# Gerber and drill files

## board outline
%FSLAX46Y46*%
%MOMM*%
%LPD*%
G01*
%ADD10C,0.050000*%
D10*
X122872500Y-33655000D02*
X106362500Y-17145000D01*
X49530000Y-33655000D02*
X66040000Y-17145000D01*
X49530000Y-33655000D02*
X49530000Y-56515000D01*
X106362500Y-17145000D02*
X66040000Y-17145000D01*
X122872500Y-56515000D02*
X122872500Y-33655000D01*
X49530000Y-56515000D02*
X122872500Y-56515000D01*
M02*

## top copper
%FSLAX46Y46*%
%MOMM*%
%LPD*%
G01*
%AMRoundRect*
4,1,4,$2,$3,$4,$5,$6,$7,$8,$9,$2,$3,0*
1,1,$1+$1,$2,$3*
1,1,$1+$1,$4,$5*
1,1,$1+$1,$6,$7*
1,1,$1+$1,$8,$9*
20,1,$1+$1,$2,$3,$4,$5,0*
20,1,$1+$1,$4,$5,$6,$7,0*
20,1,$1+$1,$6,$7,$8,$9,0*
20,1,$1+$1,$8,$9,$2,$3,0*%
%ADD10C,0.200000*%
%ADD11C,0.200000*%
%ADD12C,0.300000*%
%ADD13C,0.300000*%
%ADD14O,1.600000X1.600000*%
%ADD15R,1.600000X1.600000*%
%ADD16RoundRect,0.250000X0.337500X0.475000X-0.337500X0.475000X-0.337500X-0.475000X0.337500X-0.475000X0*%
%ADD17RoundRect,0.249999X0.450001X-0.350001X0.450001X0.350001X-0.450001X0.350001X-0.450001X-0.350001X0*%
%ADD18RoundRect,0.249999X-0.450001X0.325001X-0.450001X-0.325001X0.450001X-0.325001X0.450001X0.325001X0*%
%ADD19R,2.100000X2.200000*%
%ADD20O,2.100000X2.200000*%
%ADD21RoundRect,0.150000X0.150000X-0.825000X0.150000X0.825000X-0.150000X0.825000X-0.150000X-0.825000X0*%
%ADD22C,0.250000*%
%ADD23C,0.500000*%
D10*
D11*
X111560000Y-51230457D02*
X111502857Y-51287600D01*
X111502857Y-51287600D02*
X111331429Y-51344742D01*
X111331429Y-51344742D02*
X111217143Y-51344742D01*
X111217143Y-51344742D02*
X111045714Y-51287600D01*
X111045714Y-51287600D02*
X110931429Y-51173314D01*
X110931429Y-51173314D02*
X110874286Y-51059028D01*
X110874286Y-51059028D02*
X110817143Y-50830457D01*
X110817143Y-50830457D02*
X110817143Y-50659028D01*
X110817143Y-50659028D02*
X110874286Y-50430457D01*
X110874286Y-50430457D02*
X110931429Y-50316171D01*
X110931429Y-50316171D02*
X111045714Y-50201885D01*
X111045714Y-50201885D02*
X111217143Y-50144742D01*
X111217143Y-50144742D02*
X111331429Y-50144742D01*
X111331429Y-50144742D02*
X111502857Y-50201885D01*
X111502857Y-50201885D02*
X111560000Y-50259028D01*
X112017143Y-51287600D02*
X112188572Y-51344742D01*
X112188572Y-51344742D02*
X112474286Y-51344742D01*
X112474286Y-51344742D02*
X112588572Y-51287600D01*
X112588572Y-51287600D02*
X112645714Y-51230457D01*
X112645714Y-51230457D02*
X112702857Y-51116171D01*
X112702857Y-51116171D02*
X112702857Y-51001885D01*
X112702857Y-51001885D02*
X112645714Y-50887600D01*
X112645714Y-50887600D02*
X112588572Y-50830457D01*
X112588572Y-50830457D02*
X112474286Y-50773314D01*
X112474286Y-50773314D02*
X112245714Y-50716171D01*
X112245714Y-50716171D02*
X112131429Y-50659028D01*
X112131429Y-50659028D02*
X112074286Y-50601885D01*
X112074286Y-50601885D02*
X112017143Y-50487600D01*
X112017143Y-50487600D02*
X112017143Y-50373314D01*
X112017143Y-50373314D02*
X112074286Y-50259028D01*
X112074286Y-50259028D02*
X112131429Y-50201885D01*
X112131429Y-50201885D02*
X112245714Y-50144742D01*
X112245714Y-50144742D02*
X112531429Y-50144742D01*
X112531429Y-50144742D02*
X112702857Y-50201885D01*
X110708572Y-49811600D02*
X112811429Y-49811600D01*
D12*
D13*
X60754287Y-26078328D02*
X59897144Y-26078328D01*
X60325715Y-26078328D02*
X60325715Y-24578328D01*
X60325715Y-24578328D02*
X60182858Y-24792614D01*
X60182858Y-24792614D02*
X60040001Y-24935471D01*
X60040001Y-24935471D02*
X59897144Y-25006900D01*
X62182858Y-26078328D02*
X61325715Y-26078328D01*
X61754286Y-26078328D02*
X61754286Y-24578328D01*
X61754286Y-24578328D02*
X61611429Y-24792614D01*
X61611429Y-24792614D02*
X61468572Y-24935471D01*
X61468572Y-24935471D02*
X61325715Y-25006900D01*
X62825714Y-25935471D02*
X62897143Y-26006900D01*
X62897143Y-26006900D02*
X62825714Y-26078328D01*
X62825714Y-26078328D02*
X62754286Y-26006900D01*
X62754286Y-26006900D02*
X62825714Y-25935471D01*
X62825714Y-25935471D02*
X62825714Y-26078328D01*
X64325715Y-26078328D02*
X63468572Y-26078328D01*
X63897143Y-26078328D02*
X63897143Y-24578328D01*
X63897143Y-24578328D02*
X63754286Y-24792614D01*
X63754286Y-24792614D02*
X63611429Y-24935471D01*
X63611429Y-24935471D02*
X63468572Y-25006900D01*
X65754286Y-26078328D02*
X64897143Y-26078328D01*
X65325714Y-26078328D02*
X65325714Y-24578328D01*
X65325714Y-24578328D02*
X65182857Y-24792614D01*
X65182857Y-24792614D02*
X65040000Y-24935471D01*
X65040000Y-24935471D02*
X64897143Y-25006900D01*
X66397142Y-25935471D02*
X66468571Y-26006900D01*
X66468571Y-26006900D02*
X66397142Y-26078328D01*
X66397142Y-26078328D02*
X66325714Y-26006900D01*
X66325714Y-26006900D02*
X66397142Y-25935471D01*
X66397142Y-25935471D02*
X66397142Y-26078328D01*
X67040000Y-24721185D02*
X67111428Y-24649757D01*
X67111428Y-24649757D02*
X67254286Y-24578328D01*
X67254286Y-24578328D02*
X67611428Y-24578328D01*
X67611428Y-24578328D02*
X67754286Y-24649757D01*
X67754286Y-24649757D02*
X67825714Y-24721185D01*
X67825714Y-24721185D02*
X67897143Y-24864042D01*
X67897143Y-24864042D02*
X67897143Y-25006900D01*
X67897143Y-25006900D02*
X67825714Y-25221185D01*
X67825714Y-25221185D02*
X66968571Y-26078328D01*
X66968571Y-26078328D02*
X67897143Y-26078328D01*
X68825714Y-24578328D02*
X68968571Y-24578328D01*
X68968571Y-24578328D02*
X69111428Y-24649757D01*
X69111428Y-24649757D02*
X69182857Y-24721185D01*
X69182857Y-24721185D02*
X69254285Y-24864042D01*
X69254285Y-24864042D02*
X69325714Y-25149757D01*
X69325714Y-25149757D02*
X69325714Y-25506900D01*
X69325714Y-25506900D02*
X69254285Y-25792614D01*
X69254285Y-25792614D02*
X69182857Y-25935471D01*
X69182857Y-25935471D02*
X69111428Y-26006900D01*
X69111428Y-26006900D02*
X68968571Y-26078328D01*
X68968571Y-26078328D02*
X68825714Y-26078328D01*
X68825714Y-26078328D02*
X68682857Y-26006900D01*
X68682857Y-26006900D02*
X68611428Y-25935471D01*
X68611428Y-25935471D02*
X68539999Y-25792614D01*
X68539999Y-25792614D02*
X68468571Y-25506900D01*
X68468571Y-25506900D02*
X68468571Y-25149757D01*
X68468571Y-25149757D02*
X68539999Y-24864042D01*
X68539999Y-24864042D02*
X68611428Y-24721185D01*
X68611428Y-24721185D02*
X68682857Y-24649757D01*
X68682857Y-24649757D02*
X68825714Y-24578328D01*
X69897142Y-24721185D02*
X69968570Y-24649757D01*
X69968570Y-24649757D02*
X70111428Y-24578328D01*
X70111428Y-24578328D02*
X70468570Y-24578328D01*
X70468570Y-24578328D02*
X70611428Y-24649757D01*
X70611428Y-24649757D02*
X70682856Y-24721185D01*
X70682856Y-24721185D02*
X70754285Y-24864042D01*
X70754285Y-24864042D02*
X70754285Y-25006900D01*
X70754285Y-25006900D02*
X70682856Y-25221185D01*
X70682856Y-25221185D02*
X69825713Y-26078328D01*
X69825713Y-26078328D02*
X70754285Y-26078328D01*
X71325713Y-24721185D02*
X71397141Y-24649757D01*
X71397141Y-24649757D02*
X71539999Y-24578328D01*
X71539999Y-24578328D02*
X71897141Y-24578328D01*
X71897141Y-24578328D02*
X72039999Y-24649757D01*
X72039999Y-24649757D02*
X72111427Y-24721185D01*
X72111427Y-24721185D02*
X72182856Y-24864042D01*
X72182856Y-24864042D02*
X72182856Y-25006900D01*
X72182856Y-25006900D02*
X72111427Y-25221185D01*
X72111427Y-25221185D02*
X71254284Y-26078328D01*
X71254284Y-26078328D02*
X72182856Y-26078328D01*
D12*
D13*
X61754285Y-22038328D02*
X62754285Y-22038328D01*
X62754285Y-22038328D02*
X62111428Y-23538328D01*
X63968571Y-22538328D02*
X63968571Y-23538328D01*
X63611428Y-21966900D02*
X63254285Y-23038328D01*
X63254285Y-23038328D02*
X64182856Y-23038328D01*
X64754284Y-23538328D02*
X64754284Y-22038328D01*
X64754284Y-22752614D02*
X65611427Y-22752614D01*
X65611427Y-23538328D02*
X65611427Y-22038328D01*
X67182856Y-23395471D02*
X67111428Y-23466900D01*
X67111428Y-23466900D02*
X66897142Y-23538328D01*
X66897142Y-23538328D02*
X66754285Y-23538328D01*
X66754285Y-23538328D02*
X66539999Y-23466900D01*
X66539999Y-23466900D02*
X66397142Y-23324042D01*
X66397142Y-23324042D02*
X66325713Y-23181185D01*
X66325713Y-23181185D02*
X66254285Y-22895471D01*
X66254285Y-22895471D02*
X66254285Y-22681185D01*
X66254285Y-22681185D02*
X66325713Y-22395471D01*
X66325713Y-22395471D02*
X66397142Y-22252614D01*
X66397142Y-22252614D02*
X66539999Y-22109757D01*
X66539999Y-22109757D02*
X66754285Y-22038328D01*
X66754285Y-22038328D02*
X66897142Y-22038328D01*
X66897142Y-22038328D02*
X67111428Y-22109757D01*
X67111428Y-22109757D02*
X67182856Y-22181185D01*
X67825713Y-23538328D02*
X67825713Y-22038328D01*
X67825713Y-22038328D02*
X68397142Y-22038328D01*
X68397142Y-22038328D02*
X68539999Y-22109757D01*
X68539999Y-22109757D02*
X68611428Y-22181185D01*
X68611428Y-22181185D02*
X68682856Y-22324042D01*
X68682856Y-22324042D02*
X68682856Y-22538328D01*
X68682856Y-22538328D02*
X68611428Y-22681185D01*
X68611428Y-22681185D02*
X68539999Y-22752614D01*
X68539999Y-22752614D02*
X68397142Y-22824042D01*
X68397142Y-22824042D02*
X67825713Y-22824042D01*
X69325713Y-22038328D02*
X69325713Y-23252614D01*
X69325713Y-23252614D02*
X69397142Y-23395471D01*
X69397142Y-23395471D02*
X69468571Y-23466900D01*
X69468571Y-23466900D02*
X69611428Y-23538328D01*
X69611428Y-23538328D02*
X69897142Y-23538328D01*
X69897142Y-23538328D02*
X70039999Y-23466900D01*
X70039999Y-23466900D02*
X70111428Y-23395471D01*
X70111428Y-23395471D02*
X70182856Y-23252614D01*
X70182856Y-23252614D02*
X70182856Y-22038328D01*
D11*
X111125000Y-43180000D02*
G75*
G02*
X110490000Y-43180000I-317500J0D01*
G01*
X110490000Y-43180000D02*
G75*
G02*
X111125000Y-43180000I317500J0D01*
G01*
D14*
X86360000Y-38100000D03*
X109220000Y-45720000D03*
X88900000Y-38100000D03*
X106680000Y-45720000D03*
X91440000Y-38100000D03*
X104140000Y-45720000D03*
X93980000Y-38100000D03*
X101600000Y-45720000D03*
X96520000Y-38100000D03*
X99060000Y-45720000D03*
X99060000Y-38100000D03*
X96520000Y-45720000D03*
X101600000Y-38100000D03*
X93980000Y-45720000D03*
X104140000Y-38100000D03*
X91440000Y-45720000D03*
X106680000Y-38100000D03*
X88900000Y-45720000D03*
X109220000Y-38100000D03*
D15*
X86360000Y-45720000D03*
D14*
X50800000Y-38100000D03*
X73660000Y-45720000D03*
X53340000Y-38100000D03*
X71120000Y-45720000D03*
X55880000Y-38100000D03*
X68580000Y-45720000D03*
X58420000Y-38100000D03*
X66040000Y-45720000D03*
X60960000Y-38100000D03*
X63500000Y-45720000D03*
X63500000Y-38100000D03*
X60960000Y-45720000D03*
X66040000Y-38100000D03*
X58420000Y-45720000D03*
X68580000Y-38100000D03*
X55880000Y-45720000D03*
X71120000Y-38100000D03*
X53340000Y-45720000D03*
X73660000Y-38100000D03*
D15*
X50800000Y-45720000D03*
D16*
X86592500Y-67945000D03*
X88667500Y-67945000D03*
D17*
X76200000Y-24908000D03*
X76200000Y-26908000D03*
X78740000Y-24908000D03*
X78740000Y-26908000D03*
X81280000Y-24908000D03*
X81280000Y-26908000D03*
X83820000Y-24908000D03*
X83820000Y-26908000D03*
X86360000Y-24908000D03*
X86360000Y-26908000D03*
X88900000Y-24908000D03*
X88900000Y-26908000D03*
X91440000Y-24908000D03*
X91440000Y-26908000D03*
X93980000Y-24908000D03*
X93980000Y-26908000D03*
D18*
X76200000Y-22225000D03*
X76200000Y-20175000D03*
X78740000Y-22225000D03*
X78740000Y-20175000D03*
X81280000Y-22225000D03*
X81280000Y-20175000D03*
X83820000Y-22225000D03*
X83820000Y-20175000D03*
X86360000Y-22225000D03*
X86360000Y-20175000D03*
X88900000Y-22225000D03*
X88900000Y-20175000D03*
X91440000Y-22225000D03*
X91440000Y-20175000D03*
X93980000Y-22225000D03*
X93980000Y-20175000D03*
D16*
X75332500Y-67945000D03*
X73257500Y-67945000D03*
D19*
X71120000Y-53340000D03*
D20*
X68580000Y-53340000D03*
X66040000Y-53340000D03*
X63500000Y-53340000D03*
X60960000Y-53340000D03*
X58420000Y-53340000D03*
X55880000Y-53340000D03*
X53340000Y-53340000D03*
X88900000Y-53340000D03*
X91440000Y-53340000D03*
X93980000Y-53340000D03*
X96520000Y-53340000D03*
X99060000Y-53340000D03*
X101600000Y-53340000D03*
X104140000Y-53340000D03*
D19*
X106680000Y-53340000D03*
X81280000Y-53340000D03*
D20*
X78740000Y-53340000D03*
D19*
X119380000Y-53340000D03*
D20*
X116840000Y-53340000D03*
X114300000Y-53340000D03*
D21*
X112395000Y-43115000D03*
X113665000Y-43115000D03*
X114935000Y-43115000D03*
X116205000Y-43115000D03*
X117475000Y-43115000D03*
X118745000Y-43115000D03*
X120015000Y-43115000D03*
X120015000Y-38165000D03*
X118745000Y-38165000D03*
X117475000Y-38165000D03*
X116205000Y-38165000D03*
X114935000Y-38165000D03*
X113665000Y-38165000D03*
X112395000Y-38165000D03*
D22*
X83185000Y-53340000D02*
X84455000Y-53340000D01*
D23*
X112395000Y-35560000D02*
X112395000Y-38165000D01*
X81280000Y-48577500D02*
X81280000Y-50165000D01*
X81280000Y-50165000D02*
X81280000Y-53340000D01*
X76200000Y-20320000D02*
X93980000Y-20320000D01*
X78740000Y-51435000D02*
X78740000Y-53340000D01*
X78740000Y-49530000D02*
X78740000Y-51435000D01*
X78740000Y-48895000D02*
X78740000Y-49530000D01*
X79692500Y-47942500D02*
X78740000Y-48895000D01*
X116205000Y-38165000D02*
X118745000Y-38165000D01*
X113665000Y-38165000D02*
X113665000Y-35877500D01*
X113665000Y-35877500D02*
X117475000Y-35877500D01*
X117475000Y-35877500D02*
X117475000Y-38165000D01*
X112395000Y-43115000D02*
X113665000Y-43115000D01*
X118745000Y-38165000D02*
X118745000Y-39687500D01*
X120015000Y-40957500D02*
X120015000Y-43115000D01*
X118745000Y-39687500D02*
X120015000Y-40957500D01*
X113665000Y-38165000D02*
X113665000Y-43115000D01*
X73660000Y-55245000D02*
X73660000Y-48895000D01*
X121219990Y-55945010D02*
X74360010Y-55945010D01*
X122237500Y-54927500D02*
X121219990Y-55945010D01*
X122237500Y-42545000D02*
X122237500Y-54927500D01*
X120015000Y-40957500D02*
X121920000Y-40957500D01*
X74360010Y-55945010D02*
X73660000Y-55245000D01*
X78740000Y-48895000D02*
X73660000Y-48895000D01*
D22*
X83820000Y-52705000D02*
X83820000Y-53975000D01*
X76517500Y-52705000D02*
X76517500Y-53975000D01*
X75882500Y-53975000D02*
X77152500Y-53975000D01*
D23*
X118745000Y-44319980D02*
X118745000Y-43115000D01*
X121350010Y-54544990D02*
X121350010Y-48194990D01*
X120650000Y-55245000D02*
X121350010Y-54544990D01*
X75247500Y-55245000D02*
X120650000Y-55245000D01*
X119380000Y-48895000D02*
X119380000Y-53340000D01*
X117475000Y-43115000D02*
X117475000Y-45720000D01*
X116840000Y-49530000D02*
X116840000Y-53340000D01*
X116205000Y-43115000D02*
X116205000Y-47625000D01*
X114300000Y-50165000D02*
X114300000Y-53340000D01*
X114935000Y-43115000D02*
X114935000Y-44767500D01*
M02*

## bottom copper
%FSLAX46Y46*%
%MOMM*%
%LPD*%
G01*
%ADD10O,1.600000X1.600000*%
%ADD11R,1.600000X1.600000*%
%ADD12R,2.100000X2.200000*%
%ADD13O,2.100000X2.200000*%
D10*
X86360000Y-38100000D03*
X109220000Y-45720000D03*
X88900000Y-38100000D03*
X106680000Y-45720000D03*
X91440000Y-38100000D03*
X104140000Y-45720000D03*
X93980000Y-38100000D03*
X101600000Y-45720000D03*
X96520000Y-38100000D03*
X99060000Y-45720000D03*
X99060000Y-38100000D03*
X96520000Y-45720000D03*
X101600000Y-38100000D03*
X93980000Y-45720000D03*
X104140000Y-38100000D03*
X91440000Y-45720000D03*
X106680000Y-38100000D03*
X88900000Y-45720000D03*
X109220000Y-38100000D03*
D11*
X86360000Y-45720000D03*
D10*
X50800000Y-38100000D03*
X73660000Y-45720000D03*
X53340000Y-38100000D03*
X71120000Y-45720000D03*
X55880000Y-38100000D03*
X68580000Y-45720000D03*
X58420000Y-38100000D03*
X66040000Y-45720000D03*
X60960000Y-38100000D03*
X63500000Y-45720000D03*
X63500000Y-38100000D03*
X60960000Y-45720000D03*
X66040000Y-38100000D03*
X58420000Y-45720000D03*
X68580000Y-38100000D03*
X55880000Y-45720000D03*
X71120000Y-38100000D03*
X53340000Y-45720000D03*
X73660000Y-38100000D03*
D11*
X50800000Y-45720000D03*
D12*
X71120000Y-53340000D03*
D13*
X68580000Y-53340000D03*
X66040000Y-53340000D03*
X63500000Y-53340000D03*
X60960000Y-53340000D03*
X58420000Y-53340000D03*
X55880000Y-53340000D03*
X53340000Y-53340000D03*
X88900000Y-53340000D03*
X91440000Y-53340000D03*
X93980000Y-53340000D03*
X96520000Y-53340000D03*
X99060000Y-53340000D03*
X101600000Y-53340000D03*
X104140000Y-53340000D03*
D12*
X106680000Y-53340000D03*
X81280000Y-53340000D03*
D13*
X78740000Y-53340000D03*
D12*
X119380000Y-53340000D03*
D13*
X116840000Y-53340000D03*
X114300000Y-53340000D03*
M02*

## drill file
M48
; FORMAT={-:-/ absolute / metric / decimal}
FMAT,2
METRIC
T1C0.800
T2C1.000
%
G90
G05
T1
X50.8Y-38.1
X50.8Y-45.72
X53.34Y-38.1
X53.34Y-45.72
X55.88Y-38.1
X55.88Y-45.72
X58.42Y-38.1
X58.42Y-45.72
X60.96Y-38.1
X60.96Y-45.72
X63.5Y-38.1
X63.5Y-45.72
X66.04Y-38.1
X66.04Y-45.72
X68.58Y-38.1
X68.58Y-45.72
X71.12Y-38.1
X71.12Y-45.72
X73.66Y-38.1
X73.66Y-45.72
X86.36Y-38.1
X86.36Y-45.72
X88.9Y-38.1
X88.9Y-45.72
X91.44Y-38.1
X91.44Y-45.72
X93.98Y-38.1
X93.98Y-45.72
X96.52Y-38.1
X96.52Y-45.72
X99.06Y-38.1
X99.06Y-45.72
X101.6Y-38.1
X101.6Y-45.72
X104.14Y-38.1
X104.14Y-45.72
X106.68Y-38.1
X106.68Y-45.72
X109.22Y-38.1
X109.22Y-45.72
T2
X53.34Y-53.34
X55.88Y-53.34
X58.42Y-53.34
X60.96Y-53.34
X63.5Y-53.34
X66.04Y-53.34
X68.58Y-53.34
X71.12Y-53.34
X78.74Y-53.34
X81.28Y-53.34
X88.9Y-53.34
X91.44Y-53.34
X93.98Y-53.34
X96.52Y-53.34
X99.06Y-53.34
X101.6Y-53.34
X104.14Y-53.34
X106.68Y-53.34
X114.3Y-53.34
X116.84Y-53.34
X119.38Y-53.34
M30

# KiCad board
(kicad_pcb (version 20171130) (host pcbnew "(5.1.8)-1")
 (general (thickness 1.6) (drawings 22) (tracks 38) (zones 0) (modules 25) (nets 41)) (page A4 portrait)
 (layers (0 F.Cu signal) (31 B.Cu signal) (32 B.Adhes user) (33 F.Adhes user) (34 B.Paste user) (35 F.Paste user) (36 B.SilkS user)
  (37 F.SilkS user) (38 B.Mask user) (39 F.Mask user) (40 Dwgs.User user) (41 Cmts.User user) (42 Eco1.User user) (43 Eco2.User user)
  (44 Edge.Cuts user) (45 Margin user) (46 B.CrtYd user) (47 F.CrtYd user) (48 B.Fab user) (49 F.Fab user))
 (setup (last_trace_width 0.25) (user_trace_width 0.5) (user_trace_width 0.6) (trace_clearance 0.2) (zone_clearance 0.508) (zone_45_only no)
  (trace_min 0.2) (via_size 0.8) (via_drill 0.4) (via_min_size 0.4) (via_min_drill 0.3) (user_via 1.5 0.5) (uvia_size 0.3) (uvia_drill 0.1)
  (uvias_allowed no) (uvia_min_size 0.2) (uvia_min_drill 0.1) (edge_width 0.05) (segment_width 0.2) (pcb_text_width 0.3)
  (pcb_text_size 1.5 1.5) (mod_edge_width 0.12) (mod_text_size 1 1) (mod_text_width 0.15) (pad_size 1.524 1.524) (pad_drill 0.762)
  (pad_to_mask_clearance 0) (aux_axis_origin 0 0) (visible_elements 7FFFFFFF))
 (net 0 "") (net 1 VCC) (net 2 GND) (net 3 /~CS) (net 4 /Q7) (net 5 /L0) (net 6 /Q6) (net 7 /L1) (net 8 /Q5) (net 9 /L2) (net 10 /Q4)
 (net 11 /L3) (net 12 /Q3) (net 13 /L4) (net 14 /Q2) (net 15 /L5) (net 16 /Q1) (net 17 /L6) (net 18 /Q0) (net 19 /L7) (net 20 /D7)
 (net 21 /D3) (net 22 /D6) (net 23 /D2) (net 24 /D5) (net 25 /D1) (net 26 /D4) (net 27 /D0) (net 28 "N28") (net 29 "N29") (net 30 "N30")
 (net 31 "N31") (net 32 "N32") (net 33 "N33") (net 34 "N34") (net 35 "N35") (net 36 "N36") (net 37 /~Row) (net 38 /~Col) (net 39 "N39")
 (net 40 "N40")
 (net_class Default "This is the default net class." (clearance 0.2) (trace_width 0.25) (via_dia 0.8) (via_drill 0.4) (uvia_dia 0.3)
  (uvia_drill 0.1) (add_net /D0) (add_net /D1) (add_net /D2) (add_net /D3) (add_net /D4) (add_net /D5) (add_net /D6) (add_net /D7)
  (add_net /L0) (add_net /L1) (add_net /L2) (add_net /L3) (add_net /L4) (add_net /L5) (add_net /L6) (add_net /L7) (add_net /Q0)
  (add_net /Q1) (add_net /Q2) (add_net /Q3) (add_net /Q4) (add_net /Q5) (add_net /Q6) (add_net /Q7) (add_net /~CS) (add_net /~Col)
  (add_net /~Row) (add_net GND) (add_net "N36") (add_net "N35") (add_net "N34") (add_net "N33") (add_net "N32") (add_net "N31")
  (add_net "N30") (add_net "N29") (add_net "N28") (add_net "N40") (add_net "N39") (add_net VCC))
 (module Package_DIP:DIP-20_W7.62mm (layer F.Cu) (at 86.36 45.72 90)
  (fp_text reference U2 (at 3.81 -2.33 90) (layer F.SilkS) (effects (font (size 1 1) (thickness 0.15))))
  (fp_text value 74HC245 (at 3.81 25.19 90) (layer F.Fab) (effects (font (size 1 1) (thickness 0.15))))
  (pad 20 thru_hole oval (at 7.62 0 90) (size 1.6 1.6) (drill 0.8) (layers *.Cu *.Mask) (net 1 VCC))
  (pad 10 thru_hole oval (at 0 22.86 90) (size 1.6 1.6) (drill 0.8) (layers *.Cu *.Mask) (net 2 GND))
  (pad 19 thru_hole oval (at 7.62 2.54 90) (size 1.6 1.6) (drill 0.8) (layers *.Cu *.Mask) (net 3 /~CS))
  (pad 9 thru_hole oval (at 0 20.32 90) (size 1.6 1.6) (drill 0.8) (layers *.Cu *.Mask) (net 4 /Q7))
  (pad 18 thru_hole oval (at 7.62 5.08 90) (size 1.6 1.6) (drill 0.8) (layers *.Cu *.Mask) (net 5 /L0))
  (pad 8 thru_hole oval (at 0 17.78 90) (size 1.6 1.6) (drill 0.8) (layers *.Cu *.Mask) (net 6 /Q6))
  (pad 17 thru_hole oval (at 7.62 7.62 90) (size 1.6 1.6) (drill 0.8) (layers *.Cu *.Mask) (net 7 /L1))
  (pad 7 thru_hole oval (at 0 15.24 90) (size 1.6 1.6) (drill 0.8) (layers *.Cu *.Mask) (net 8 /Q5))
  (pad 16 thru_hole oval (at 7.62 10.16 90) (size 1.6 1.6) (drill 0.8) (layers *.Cu *.Mask) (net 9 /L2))
  (pad 6 thru_hole oval (at 0 12.7 90) (size 1.6 1.6) (drill 0.8) (layers *.Cu *.Mask) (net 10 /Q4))
  (pad 15 thru_hole oval (at 7.62 12.7 90) (size 1.6 1.6) (drill 0.8) (layers *.Cu *.Mask) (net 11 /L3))
  (pad 5 thru_hole oval (at 0 10.16 90) (size 1.6 1.6) (drill 0.8) (layers *.Cu *.Mask) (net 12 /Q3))
  (pad 14 thru_hole oval (at 7.62 15.24 90) (size 1.6 1.6) (drill 0.8) (layers *.Cu *.Mask) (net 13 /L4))
  (pad 4 thru_hole oval (at 0 7.62 90) (size 1.6 1.6) (drill 0.8) (layers *.Cu *.Mask) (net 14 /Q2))
  (pad 13 thru_hole oval (at 7.62 17.78 90) (size 1.6 1.6) (drill 0.8) (layers *.Cu *.Mask) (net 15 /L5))
  (pad 3 thru_hole oval (at 0 5.08 90) (size 1.6 1.6) (drill 0.8) (layers *.Cu *.Mask) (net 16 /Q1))
  (pad 12 thru_hole oval (at 7.62 20.32 90) (size 1.6 1.6) (drill 0.8) (layers *.Cu *.Mask) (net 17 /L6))
  (pad 2 thru_hole oval (at 0 2.54 90) (size 1.6 1.6) (drill 0.8) (layers *.Cu *.Mask) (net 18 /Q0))
  (pad 11 thru_hole oval (at 7.62 22.86 90) (size 1.6 1.6) (drill 0.8) (layers *.Cu *.Mask) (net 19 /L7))
  (pad 1 thru_hole rect (at 0 0 90) (size 1.6 1.6) (drill 0.8) (layers *.Cu *.Mask) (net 2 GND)))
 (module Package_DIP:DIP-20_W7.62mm (layer F.Cu) (at 50.8 45.72 90)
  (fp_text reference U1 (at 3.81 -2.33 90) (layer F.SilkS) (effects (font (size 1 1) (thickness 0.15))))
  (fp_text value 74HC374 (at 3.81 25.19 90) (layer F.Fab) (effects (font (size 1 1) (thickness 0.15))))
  (pad 20 thru_hole oval (at 7.62 0 90) (size 1.6 1.6) (drill 0.8) (layers *.Cu *.Mask) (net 1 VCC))
  (pad 10 thru_hole oval (at 0 22.86 90) (size 1.6 1.6) (drill 0.8) (layers *.Cu *.Mask) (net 2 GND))
  (pad 19 thru_hole oval (at 7.62 2.54 90) (size 1.6 1.6) (drill 0.8) (layers *.Cu *.Mask) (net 19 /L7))
  (pad 9 thru_hole oval (at 0 20.32 90) (size 1.6 1.6) (drill 0.8) (layers *.Cu *.Mask) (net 11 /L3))
  (pad 18 thru_hole oval (at 7.62 5.08 90) (size 1.6 1.6) (drill 0.8) (layers *.Cu *.Mask) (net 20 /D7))
  (pad 8 thru_hole oval (at 0 17.78 90) (size 1.6 1.6) (drill 0.8) (layers *.Cu *.Mask) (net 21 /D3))
  (pad 17 thru_hole oval (at 7.62 7.62 90) (size 1.6 1.6) (drill 0.8) (layers *.Cu *.Mask) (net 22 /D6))
  (pad 7 thru_hole oval (at 0 15.24 90) (size 1.6 1.6) (drill 0.8) (layers *.Cu *.Mask) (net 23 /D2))
  (pad 16 thru_hole oval (at 7.62 10.16 90) (size 1.6 1.6) (drill 0.8) (layers *.Cu *.Mask) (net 17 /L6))
  (pad 6 thru_hole oval (at 0 12.7 90) (size 1.6 1.6) (drill 0.8) (layers *.Cu *.Mask) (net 9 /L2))
  (pad 15 thru_hole oval (at 7.62 12.7 90) (size 1.6 1.6) (drill 0.8) (layers *.Cu *.Mask) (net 15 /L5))
  (pad 5 thru_hole oval (at 0 10.16 90) (size 1.6 1.6) (drill 0.8) (layers *.Cu *.Mask) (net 7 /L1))
  (pad 14 thru_hole oval (at 7.62 15.24 90) (size 1.6 1.6) (drill 0.8) (layers *.Cu *.Mask) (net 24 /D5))
  (pad 4 thru_hole oval (at 0 7.62 90) (size 1.6 1.6) (drill 0.8) (layers *.Cu *.Mask) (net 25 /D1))
  (pad 13 thru_hole oval (at 7.62 17.78 90) (size 1.6 1.6) (drill 0.8) (layers *.Cu *.Mask) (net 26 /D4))
  (pad 3 thru_hole oval (at 0 5.08 90) (size 1.6 1.6) (drill 0.8) (layers *.Cu *.Mask) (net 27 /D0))
  (pad 12 thru_hole oval (at 7.62 20.32 90) (size 1.6 1.6) (drill 0.8) (layers *.Cu *.Mask) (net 13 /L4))
  (pad 2 thru_hole oval (at 0 2.54 90) (size 1.6 1.6) (drill 0.8) (layers *.Cu *.Mask) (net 5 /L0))
  (pad 11 thru_hole oval (at 7.62 22.86 90) (size 1.6 1.6) (drill 0.8) (layers *.Cu *.Mask) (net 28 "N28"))
  (pad 1 thru_hole rect (at 0 0 90) (size 1.6 1.6) (drill 0.8) (layers *.Cu *.Mask) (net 2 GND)))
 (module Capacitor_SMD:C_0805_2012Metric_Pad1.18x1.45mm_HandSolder (layer F.Cu) (at 87.63 67.945 180)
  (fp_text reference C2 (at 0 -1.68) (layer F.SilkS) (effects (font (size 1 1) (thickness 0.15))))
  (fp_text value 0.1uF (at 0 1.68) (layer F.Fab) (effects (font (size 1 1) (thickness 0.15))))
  (pad 2 smd roundrect (at 1.0375 0 180) (size 1.175 1.45) (layers F.Cu F.Paste F.Mask) (roundrect_rratio 0.2127659574468085) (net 2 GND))
  (pad 1 smd roundrect (at -1.0375 0 180) (size 1.175 1.45) (layers F.Cu F.Paste F.Mask) (roundrect_rratio 0.2127659574468085) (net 1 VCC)))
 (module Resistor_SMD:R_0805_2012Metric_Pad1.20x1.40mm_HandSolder (layer F.Cu) (at 76.2 25.908 90)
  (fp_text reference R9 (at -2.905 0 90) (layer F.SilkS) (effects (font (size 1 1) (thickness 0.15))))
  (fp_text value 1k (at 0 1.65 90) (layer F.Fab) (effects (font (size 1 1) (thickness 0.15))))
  (pad 2 smd roundrect (at 1 0 90) (size 1.2 1.4) (layers F.Cu F.Paste F.Mask) (roundrect_rratio 0.2083325) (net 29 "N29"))
  (pad 1 smd roundrect (at -1 0 90) (size 1.2 1.4) (layers F.Cu F.Paste F.Mask) (roundrect_rratio 0.2083325) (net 19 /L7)))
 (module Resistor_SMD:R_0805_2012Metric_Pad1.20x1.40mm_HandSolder (layer F.Cu) (at 78.74 25.908 90)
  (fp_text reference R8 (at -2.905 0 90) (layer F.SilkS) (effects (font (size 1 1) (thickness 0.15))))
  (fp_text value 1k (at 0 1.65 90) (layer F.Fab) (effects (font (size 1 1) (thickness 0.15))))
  (pad 2 smd roundrect (at 1 0 90) (size 1.2 1.4) (layers F.Cu F.Paste F.Mask) (roundrect_rratio 0.2083325) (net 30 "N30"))
  (pad 1 smd roundrect (at -1 0 90) (size 1.2 1.4) (layers F.Cu F.Paste F.Mask) (roundrect_rratio 0.2083325) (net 17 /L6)))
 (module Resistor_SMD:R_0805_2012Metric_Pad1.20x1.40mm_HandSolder (layer F.Cu) (at 81.28 25.908 90)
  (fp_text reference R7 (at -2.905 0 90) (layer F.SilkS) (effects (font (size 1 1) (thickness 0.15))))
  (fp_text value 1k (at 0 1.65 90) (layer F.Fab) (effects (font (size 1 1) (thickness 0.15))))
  (pad 2 smd roundrect (at 1 0 90) (size 1.2 1.4) (layers F.Cu F.Paste F.Mask) (roundrect_rratio 0.2083325) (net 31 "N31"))
  (pad 1 smd roundrect (at -1 0 90) (size 1.2 1.4) (layers F.Cu F.Paste F.Mask) (roundrect_rratio 0.2083325) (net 15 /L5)))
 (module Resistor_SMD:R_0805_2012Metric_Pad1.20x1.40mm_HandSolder (layer F.Cu) (at 83.82 25.908 90)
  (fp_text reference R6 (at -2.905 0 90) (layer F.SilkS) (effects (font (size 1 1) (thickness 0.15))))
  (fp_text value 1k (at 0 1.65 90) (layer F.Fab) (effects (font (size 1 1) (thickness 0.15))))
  (pad 2 smd roundrect (at 1 0 90) (size 1.2 1.4) (layers F.Cu F.Paste F.Mask) (roundrect_rratio 0.2083325) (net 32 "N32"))
  (pad 1 smd roundrect (at -1 0 90) (size 1.2 1.4) (layers F.Cu F.Paste F.Mask) (roundrect_rratio 0.2083325) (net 13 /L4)))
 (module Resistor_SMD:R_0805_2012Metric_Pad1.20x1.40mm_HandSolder (layer F.Cu) (at 86.36 25.908 90)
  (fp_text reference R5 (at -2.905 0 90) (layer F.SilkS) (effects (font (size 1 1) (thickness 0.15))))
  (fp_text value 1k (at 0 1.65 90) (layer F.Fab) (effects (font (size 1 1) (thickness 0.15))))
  (pad 2 smd roundrect (at 1 0 90) (size 1.2 1.4) (layers F.Cu F.Paste F.Mask) (roundrect_rratio 0.2083325) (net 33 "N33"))
  (pad 1 smd roundrect (at -1 0 90) (size 1.2 1.4) (layers F.Cu F.Paste F.Mask) (roundrect_rratio 0.2083325) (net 11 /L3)))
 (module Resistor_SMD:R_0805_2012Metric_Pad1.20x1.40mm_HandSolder (layer F.Cu) (at 88.9 25.908 90)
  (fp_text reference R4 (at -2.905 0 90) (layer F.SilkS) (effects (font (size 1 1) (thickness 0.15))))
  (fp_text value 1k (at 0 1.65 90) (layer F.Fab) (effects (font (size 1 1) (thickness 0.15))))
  (pad 2 smd roundrect (at 1 0 90) (size 1.2 1.4) (layers F.Cu F.Paste F.Mask) (roundrect_rratio 0.2083325) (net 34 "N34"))
  (pad 1 smd roundrect (at -1 0 90) (size 1.2 1.4) (layers F.Cu F.Paste F.Mask) (roundrect_rratio 0.2083325) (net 9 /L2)))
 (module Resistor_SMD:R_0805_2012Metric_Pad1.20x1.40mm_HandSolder (layer F.Cu) (at 91.44 25.908 90)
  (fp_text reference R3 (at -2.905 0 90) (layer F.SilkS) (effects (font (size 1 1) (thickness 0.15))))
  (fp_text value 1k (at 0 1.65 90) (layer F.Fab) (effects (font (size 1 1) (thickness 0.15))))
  (pad 2 smd roundrect (at 1 0 90) (size 1.2 1.4) (layers F.Cu F.Paste F.Mask) (roundrect_rratio 0.2083325) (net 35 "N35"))
  (pad 1 smd roundrect (at -1 0 90) (size 1.2 1.4) (layers F.Cu F.Paste F.Mask) (roundrect_rratio 0.2083325) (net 7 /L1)))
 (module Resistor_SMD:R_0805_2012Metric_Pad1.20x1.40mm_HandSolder (layer F.Cu) (at 93.98 25.908 90)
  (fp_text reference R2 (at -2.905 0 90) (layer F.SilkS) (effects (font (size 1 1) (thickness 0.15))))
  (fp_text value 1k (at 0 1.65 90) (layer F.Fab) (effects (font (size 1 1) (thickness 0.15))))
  (pad 2 smd roundrect (at 1 0 90) (size 1.2 1.4) (layers F.Cu F.Paste F.Mask) (roundrect_rratio 0.2083325) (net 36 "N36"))
  (pad 1 smd roundrect (at -1 0 90) (size 1.2 1.4) (layers F.Cu F.Paste F.Mask) (roundrect_rratio 0.2083325) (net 5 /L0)))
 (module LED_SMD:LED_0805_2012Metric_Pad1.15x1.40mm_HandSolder (layer F.Cu) (at 76.2 21.2 270)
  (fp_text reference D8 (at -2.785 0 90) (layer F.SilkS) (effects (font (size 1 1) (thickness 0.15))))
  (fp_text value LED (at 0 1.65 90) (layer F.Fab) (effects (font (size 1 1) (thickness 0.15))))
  (pad 2 smd roundrect (at 1.025 0 270) (size 1.15 1.4) (layers F.Cu F.Paste F.Mask) (roundrect_rratio 0.2173904347826087) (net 29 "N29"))
  (pad 1 smd roundrect (at -1.025 0 270) (size 1.15 1.4) (layers F.Cu F.Paste F.Mask) (roundrect_rratio 0.2173904347826087) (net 2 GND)))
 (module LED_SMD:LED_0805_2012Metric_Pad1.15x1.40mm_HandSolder (layer F.Cu) (at 78.74 21.2 270)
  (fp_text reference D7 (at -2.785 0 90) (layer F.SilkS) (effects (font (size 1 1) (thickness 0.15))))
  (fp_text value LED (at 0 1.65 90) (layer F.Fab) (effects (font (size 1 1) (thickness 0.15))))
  (pad 2 smd roundrect (at 1.025 0 270) (size 1.15 1.4) (layers F.Cu F.Paste F.Mask) (roundrect_rratio 0.2173904347826087) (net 30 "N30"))
  (pad 1 smd roundrect (at -1.025 0 270) (size 1.15 1.4) (layers F.Cu F.Paste F.Mask) (roundrect_rratio 0.2173904347826087) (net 2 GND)))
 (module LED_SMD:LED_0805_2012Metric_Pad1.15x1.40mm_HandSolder (layer F.Cu) (at 81.28 21.2 270)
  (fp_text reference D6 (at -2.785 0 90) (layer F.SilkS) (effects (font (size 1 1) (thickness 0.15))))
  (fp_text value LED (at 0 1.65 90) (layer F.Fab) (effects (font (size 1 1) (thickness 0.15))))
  (pad 2 smd roundrect (at 1.025 0 270) (size 1.15 1.4) (layers F.Cu F.Paste F.Mask) (roundrect_rratio 0.2173904347826087) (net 31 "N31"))
  (pad 1 smd roundrect (at -1.025 0 270) (size 1.15 1.4) (layers F.Cu F.Paste F.Mask) (roundrect_rratio 0.2173904347826087) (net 2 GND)))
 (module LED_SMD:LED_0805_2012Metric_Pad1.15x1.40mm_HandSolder (layer F.Cu) (at 83.82 21.2 270)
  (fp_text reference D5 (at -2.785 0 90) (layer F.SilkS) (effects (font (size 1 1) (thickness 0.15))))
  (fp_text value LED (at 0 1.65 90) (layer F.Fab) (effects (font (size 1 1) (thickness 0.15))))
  (pad 2 smd roundrect (at 1.025 0 270) (size 1.15 1.4) (layers F.Cu F.Paste F.Mask) (roundrect_rratio 0.2173904347826087) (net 32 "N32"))
  (pad 1 smd roundrect (at -1.025 0 270) (size 1.15 1.4) (layers F.Cu F.Paste F.Mask) (roundrect_rratio 0.2173904347826087) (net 2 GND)))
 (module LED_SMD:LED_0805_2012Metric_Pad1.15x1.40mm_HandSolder (layer F.Cu) (at 86.36 21.2 270)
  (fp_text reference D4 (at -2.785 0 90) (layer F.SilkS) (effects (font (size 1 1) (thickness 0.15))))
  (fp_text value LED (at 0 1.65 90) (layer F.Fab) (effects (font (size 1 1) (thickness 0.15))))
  (pad 2 smd roundrect (at 1.025 0 270) (size 1.15 1.4) (layers F.Cu F.Paste F.Mask) (roundrect_rratio 0.2173904347826087) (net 33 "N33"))
  (pad 1 smd roundrect (at -1.025 0 270) (size 1.15 1.4) (layers F.Cu F.Paste F.Mask) (roundrect_rratio 0.2173904347826087) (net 2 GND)))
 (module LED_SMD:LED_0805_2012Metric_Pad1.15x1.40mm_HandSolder (layer F.Cu) (at 88.9 21.2 270)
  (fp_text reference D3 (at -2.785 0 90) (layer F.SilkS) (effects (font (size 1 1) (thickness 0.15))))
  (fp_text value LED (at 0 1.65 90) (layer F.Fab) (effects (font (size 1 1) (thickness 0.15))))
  (pad 2 smd roundrect (at 1.025 0 270) (size 1.15 1.4) (layers F.Cu F.Paste F.Mask) (roundrect_rratio 0.2173904347826087) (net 34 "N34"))
  (pad 1 smd roundrect (at -1.025 0 270) (size 1.15 1.4) (layers F.Cu F.Paste F.Mask) (roundrect_rratio 0.2173904347826087) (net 2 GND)))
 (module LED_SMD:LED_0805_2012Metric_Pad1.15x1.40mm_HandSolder (layer F.Cu) (at 91.44 21.2 270)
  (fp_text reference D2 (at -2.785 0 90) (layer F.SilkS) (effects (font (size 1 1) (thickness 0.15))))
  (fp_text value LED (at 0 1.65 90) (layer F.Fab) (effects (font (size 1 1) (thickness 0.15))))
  (pad 2 smd roundrect (at 1.025 0 270) (size 1.15 1.4) (layers F.Cu F.Paste F.Mask) (roundrect_rratio 0.2173904347826087) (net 35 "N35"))
  (pad 1 smd roundrect (at -1.025 0 270) (size 1.15 1.4) (layers F.Cu F.Paste F.Mask) (roundrect_rratio 0.2173904347826087) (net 2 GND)))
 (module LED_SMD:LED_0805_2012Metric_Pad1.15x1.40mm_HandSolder (layer F.Cu) (at 93.98 21.2 270)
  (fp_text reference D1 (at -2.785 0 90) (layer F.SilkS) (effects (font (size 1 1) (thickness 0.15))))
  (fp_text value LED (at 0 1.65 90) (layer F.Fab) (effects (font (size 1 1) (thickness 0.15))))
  (pad 2 smd roundrect (at 1.025 0 270) (size 1.15 1.4) (layers F.Cu F.Paste F.Mask) (roundrect_rratio 0.2173904347826087) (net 36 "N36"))
  (pad 1 smd roundrect (at -1.025 0 270) (size 1.15 1.4) (layers F.Cu F.Paste F.Mask) (roundrect_rratio 0.2173904347826087) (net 2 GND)))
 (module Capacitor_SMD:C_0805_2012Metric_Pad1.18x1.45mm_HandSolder (layer F.Cu) (at 74.295 67.945 180)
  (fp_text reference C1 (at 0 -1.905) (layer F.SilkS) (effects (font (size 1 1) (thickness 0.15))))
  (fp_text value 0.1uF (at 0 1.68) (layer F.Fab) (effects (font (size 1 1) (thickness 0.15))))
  (pad 1 smd roundrect (at -1.0375 0 180) (size 1.175 1.45) (layers F.Cu F.Paste F.Mask) (roundrect_rratio 0.2127659574468085) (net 1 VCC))
  (pad 2 smd roundrect (at 1.0375 0 180) (size 1.175 1.45) (layers F.Cu F.Paste F.Mask) (roundrect_rratio 0.2127659574468085) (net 2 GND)))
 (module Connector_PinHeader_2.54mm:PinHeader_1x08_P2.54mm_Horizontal (layer F.Cu) (at 71.12 53.34 270)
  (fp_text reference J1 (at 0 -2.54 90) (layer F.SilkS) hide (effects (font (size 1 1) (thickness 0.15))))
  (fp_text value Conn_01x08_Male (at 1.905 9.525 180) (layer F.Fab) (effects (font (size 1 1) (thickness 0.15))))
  (pad 1 thru_hole rect (at 0 0 270) (size 2.2 2.1) (drill 1) (layers *.Cu *.Mask) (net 27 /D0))
  (pad 2 thru_hole oval (at 0 2.54 270) (size 2.2 2.1) (drill 1) (layers *.Cu *.Mask) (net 25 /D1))
  (pad 3 thru_hole oval (at 0 5.08 270) (size 2.2 2.1) (drill 1) (layers *.Cu *.Mask) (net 23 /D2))
  (pad 4 thru_hole oval (at 0 7.62 270) (size 2.2 2.1) (drill 1) (layers *.Cu *.Mask) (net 21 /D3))
  (pad 5 thru_hole oval (at 0 10.16 270) (size 2.2 2.1) (drill 1) (layers *.Cu *.Mask) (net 26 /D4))
  (pad 6 thru_hole oval (at 0 12.7 270) (size 2.2 2.1) (drill 1) (layers *.Cu *.Mask) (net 24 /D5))
  (pad 7 thru_hole oval (at 0 15.24 270) (size 2.2 2.1) (drill 1) (layers *.Cu *.Mask) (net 22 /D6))
  (pad 8 thru_hole oval (at 0 17.78 270) (size 2.2 2.1) (drill 1) (layers *.Cu *.Mask) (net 20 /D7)))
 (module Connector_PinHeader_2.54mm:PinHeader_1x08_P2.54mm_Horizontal (layer F.Cu) (at 106.68 53.34 270)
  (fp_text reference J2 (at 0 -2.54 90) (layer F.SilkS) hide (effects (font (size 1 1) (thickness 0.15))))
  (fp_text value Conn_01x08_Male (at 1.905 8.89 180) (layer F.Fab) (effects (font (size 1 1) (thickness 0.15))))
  (pad 8 thru_hole oval (at 0 17.78 270) (size 2.2 2.1) (drill 1) (layers *.Cu *.Mask) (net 18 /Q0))
  (pad 7 thru_hole oval (at 0 15.24 270) (size 2.2 2.1) (drill 1) (layers *.Cu *.Mask) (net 16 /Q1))
  (pad 6 thru_hole oval (at 0 12.7 270) (size 2.2 2.1) (drill 1) (layers *.Cu *.Mask) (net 14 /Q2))
  (pad 5 thru_hole oval (at 0 10.16 270) (size 2.2 2.1) (drill 1) (layers *.Cu *.Mask) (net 12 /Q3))
  (pad 4 thru_hole oval (at 0 7.62 270) (size 2.2 2.1) (drill 1) (layers *.Cu *.Mask) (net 10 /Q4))
  (pad 3 thru_hole oval (at 0 5.08 270) (size 2.2 2.1) (drill 1) (layers *.Cu *.Mask) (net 8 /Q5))
  (pad 2 thru_hole oval (at 0 2.54 270) (size 2.2 2.1) (drill 1) (layers *.Cu *.Mask) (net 6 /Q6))
  (pad 1 thru_hole rect (at 0 0 270) (size 2.2 2.1) (drill 1) (layers *.Cu *.Mask) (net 4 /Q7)))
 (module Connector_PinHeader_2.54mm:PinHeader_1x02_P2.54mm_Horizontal (layer F.Cu) (at 81.28 53.34 270)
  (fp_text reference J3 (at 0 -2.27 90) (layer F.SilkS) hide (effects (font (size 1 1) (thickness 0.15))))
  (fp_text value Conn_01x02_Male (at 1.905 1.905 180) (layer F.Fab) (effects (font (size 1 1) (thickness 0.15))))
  (pad 1 thru_hole rect (at 0 0 270) (size 2.2 2.1) (drill 1) (layers *.Cu *.Mask) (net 1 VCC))
  (pad 2 thru_hole oval (at 0 2.54 270) (size 2.2 2.1) (drill 1) (layers *.Cu *.Mask) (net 2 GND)))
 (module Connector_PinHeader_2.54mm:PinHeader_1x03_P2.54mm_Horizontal (layer F.Cu) (at 119.38 53.34 270)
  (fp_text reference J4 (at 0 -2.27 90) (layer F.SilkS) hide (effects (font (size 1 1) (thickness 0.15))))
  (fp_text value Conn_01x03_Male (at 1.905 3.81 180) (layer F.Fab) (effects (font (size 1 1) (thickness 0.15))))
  (pad 1 thru_hole rect (at 0 0 270) (size 2.2 2.1) (drill 1) (layers *.Cu *.Mask) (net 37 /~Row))
  (pad 2 thru_hole oval (at 0 2.54 270) (size 2.2 2.1) (drill 1) (layers *.Cu *.Mask) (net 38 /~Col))
  (pad 3 thru_hole oval (at 0 5.08 270) (size 2.2 2.1) (drill 1) (layers *.Cu *.Mask) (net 3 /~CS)))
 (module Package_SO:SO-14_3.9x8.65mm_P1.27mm (layer F.Cu) (at 116.205 40.64 90)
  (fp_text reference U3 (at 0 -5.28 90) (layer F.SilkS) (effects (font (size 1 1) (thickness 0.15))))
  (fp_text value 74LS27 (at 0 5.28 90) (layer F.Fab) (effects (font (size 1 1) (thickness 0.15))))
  (pad 1 smd roundrect (at -2.475 -3.81 90) (size 1.95 0.6) (layers F.Cu F.Paste F.Mask) (roundrect_rratio 0.25) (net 2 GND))
  (pad 2 smd roundrect (at -2.475 -2.54 90) (size 1.95 0.6) (layers F.Cu F.Paste F.Mask) (roundrect_rratio 0.25) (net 2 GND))
  (pad 3 smd roundrect (at -2.475 -1.27 90) (size 1.95 0.6) (layers F.Cu F.Paste F.Mask) (roundrect_rratio 0.25) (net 3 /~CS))
  (pad 4 smd roundrect (at -2.475 0 90) (size 1.95 0.6) (layers F.Cu F.Paste F.Mask) (roundrect_rratio 0.25) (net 38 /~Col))
  (pad 5 smd roundrect (at -2.475 1.27 90) (size 1.95 0.6) (layers F.Cu F.Paste F.Mask) (roundrect_rratio 0.25) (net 37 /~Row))
  (pad 6 smd roundrect (at -2.475 2.54 90) (size 1.95 0.6) (layers F.Cu F.Paste F.Mask) (roundrect_rratio 0.25) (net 28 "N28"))
  (pad 7 smd roundrect (at -2.475 3.81 90) (size 1.95 0.6) (layers F.Cu F.Paste F.Mask) (roundrect_rratio 0.25) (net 2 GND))
  (pad 8 smd roundrect (at 2.475 3.81 90) (size 1.95 0.6) (layers F.Cu F.Paste F.Mask) (roundrect_rratio 0.25) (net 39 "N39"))
  (pad 9 smd roundrect (at 2.475 2.54 90) (size 1.95 0.6) (layers F.Cu F.Paste F.Mask) (roundrect_rratio 0.25) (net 2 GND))
  (pad 10 smd roundrect (at 2.475 1.27 90) (size 1.95 0.6) (layers F.Cu F.Paste F.Mask) (roundrect_rratio 0.25) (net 2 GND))
  (pad 11 smd roundrect (at 2.475 0 90) (size 1.95 0.6) (layers F.Cu F.Paste F.Mask) (roundrect_rratio 0.25) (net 2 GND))
  (pad 12 smd roundrect (at 2.475 -1.27 90) (size 1.95 0.6) (layers F.Cu F.Paste F.Mask) (roundrect_rratio 0.25) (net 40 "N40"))
  (pad 13 smd roundrect (at 2.475 -2.54 90) (size 1.95 0.6) (layers F.Cu F.Paste F.Mask) (roundrect_rratio 0.25) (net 2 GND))
  (pad 14 smd roundrect (at 2.475 -3.81 90) (size 1.95 0.6) (layers F.Cu F.Paste F.Mask) (roundrect_rratio 0.25) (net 1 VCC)))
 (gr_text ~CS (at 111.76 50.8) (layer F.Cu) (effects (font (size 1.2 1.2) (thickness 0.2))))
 (gr_line (start 122.8725 33.655) (end 106.3625 17.145) (layer Edge.Cuts) (width 0.05))
 (gr_line (start 49.53 33.655) (end 66.04 17.145) (layer Edge.Cuts) (width 0.05))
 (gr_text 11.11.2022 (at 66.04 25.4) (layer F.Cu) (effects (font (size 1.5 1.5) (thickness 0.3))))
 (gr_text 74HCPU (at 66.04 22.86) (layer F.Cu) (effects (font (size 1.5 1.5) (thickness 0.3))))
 (gr_circle (center 110.8075 43.18) (end 111.125 43.18) (layer F.Cu) (width 0.2))
 (gr_line (start 49.53 33.655) (end 49.53 56.515) (layer Edge.Cuts) (width 0.05))
 (gr_line (start 106.3625 17.145) (end 66.04 17.145) (layer Edge.Cuts) (width 0.05))
 (gr_line (start 122.8725 56.515) (end 122.8725 33.655) (layer Edge.Cuts) (width 0.05))
 (gr_line (start 49.53 56.515) (end 122.8725 56.515) (layer Edge.Cuts) (width 0.05))
 (segment (start 83.185 53.34) (end 84.455 53.34) (width 0.25) (layer F.Cu) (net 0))
 (segment (start 112.395 35.56) (end 112.395 38.165) (width 0.5) (layer F.Cu) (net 1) (status 20))
 (segment (start 81.28 48.5775) (end 81.28 50.165) (width 0.5) (layer F.Cu) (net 1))
 (segment (start 81.28 50.165) (end 81.28 53.34) (width 0.5) (layer F.Cu) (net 1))
 (segment (start 76.2 20.32) (end 93.98 20.32) (width 0.5) (layer F.Cu) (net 2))
 (segment (start 78.74 51.435) (end 78.74 53.34) (width 0.5) (layer F.Cu) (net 2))
 (segment (start 78.74 49.53) (end 78.74 51.435) (width 0.5) (layer F.Cu) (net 2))
 (segment (start 78.74 48.895) (end 78.74 49.53) (width 0.5) (layer F.Cu) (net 2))
 (segment (start 79.6925 47.9425) (end 78.74 48.895) (width 0.5) (layer F.Cu) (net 2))
 (segment (start 116.205 38.165) (end 118.745 38.165) (width 0.5) (layer F.Cu) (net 2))
 (segment (start 113.665 38.165) (end 113.665 35.8775) (width 0.5) (layer F.Cu) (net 2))
 (segment (start 113.665 35.8775) (end 117.475 35.8775) (width 0.5) (layer F.Cu) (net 2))
 (segment (start 117.475 35.8775) (end 117.475 38.165) (width 0.5) (layer F.Cu) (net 2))
 (segment (start 112.395 43.115) (end 113.665 43.115) (width 0.5) (layer F.Cu) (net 2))
 (segment (start 118.745 38.165) (end 118.745 39.6875) (width 0.5) (layer F.Cu) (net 2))
 (segment (start 120.015 40.9575) (end 120.015 43.115) (width 0.5) (layer F.Cu) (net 2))
 (segment (start 118.745 39.6875) (end 120.015 40.9575) (width 0.5) (layer F.Cu) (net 2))
 (segment (start 113.665 38.165) (end 113.665 43.115) (width 0.5) (layer F.Cu) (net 2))
 (segment (start 73.66 55.245) (end 73.66 48.895) (width 0.5) (layer F.Cu) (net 2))
 (segment (start 121.21999 55.94501) (end 74.36001 55.94501) (width 0.5) (layer F.Cu) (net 2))
 (segment (start 122.2375 54.9275) (end 121.21999 55.94501) (width 0.5) (layer F.Cu) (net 2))
 (segment (start 122.2375 42.545) (end 122.2375 54.9275) (width 0.5) (layer F.Cu) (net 2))
 (segment (start 120.015 40.9575) (end 121.92 40.9575) (width 0.5) (layer F.Cu) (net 2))
 (segment (start 74.36001 55.94501) (end 73.66 55.245) (width 0.5) (layer F.Cu) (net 2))
 (segment (start 78.74 48.895) (end 73.66 48.895) (width 0.5) (layer F.Cu) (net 2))
 (segment (start 83.82 52.705) (end 83.82 53.975) (width 0.25) (layer F.Cu) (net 24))
 (segment (start 76.5175 52.705) (end 76.5175 53.975) (width 0.25) (layer F.Cu) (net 23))
 (segment (start 75.8825 53.975) (end 77.1525 53.975) (width 0.25) (layer F.Cu) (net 23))
 (segment (start 118.745 44.31998) (end 118.745 43.115) (width 0.5) (layer F.Cu) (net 28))
 (segment (start 121.35001 54.54499) (end 121.35001 48.19499) (width 0.5) (layer F.Cu) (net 28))
 (segment (start 120.65 55.245) (end 121.35001 54.54499) (width 0.5) (layer F.Cu) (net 28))
 (segment (start 75.2475 55.245) (end 120.65 55.245) (width 0.5) (layer F.Cu) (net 28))
 (segment (start 119.38 48.895) (end 119.38 53.34) (width 0.5) (layer F.Cu) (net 37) (status 20))
 (segment (start 117.475 43.115) (end 117.475 45.72) (width 0.5) (layer F.Cu) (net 37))
 (segment (start 116.84 49.53) (end 116.84 53.34) (width 0.5) (layer F.Cu) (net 38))
 (segment (start 116.205 43.115) (end 116.205 47.625) (width 0.5) (layer F.Cu) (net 38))
 (segment (start 114.3 50.165) (end 114.3 53.34) (width 0.5) (layer F.Cu) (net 3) (status 20))
 (segment (start 114.935 43.115) (end 114.935 44.7675) (width 0.5) (layer F.Cu) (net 3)))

